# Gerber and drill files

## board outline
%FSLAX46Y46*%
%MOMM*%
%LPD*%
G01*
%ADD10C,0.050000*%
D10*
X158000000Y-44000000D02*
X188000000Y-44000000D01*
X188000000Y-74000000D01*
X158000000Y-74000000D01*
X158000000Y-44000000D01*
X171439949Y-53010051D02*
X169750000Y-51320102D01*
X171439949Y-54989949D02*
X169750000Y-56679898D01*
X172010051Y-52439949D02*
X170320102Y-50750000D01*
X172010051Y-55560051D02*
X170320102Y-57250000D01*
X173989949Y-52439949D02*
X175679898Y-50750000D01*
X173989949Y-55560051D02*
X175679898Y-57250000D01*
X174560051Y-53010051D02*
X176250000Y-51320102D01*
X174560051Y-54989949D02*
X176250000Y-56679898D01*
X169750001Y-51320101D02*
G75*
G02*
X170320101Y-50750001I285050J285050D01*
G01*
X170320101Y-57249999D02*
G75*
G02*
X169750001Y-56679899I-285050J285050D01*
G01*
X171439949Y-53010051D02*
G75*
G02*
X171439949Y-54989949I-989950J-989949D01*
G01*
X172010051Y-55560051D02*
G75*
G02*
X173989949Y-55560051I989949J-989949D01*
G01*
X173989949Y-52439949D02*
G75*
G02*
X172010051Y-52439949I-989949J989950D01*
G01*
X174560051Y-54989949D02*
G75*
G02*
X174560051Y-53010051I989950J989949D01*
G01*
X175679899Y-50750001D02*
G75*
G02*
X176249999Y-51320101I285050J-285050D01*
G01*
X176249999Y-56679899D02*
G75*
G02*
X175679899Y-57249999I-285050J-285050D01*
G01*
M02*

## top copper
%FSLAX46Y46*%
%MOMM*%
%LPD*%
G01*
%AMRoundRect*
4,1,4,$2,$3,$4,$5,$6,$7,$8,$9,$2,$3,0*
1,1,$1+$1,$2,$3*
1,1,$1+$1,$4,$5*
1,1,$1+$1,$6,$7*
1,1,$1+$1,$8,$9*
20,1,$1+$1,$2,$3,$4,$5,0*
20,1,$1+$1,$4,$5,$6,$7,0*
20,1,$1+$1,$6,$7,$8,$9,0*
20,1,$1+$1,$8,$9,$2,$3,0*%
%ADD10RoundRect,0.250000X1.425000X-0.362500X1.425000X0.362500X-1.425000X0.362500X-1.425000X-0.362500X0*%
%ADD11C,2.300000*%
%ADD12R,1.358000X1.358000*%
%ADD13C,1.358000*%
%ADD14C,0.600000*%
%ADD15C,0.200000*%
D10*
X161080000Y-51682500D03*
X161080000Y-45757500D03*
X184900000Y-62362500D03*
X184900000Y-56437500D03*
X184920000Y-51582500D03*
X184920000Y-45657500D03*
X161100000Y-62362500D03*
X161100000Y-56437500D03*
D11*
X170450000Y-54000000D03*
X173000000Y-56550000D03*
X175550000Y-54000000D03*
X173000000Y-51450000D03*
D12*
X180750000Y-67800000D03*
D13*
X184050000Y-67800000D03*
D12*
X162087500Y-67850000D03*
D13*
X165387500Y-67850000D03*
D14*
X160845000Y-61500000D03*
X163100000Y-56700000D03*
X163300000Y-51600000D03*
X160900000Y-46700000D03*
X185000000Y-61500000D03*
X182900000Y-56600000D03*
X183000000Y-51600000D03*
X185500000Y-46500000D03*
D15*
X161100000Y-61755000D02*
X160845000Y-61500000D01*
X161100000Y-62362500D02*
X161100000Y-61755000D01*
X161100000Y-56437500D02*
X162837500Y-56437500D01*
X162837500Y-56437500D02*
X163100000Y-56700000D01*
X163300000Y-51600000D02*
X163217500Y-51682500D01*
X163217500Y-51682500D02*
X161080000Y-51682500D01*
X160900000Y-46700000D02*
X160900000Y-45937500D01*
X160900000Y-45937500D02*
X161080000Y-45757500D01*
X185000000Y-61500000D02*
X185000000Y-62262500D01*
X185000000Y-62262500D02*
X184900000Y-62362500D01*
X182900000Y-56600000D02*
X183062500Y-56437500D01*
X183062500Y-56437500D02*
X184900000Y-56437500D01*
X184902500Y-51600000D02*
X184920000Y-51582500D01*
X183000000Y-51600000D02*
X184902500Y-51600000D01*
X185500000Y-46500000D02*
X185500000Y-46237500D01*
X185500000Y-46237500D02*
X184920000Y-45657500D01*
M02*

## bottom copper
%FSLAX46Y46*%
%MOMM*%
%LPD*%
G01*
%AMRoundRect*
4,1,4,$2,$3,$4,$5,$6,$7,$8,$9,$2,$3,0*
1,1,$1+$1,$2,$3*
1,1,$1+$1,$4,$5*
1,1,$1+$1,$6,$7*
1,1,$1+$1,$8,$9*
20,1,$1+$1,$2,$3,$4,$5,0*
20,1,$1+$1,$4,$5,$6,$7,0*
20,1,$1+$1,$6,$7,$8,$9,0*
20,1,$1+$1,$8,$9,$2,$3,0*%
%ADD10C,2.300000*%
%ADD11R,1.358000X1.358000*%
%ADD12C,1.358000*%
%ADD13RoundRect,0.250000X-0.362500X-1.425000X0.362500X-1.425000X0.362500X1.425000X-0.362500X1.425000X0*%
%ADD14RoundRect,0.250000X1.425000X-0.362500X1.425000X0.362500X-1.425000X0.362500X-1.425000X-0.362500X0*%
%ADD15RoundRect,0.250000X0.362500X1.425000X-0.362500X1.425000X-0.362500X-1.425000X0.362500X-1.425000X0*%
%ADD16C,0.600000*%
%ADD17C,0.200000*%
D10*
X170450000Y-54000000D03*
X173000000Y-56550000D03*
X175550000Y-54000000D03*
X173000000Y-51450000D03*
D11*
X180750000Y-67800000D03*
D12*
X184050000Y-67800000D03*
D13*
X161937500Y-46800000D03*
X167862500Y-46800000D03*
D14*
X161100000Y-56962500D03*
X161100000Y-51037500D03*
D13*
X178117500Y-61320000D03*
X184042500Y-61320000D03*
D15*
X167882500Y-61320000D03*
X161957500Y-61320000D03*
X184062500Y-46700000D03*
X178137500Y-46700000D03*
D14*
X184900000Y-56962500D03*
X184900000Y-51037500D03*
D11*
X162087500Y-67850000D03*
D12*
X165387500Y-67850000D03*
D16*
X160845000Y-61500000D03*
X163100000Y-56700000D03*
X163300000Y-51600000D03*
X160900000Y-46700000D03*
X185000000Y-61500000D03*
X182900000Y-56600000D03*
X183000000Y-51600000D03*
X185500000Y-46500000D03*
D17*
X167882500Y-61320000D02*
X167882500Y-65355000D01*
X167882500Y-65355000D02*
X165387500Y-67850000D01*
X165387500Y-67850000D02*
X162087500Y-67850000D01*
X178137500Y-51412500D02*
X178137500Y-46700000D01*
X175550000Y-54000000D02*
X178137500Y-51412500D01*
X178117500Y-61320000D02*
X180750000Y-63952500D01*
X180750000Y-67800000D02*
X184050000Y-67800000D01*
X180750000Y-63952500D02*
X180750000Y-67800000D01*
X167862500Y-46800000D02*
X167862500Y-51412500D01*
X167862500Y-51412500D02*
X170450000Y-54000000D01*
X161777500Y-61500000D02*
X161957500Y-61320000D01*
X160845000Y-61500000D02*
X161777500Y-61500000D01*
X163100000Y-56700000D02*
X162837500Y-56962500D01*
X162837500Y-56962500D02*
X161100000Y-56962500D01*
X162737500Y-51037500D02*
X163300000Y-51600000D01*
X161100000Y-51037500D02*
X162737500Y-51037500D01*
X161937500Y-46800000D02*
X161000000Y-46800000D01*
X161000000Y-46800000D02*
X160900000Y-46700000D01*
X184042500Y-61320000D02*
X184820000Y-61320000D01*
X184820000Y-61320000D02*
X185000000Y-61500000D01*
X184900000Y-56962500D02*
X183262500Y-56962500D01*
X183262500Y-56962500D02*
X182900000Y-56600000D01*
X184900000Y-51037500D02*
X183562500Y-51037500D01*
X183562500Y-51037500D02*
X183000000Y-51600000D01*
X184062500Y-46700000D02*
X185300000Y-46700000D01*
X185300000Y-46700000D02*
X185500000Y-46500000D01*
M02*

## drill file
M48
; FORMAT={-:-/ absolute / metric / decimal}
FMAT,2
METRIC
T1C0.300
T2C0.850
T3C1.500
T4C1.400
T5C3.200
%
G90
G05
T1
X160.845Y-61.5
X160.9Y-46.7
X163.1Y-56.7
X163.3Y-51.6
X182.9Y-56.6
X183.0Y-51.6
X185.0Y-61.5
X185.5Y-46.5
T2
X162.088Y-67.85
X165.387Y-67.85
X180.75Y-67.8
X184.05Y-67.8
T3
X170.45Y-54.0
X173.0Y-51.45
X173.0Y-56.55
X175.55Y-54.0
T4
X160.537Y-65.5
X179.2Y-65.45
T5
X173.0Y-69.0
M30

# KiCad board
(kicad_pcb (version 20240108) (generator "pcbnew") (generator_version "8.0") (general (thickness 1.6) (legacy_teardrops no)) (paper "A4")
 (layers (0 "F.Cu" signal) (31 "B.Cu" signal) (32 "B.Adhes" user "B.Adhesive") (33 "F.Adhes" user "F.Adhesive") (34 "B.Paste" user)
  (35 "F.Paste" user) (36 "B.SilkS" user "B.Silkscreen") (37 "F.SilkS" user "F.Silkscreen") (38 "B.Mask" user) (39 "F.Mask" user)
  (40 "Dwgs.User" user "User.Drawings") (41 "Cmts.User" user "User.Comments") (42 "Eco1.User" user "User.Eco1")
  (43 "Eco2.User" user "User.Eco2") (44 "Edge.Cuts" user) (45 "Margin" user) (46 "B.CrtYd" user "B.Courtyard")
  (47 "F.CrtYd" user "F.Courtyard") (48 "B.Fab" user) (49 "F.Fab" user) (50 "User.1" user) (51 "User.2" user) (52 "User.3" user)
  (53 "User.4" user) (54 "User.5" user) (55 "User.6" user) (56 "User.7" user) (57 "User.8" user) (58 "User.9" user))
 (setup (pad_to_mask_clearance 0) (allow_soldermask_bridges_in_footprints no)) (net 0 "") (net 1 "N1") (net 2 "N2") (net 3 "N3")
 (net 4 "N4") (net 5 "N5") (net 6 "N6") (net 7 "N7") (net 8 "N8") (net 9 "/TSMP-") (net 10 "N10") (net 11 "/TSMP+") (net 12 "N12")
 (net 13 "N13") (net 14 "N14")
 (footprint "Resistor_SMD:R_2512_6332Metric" (layer "F.Cu") (at 161.08 48.72 90)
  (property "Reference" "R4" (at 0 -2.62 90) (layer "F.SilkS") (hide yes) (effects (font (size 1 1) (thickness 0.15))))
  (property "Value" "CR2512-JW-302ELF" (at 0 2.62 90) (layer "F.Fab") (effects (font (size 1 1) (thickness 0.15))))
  (pad "1" smd roundrect (at -2.9625 0 90) (size 1.225 3.35) (layers "F.Cu" "F.Paste" "F.Mask") (roundrect_rratio 0.204082) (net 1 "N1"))
  (pad "2" smd roundrect (at 2.9625 0 90) (size 1.225 3.35) (layers "F.Cu" "F.Paste" "F.Mask") (roundrect_rratio 0.204082) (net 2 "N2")))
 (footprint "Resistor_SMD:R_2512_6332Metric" (layer "F.Cu") (at 184.9 59.4 90)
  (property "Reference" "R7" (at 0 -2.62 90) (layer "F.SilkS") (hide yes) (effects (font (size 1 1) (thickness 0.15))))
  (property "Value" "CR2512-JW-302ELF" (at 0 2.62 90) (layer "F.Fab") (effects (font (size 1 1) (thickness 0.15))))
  (pad "1" smd roundrect (at -2.9625 0 90) (size 1.225 3.35) (layers "F.Cu" "F.Paste" "F.Mask") (roundrect_rratio 0.204082) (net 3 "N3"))
  (pad "2" smd roundrect (at 2.9625 0 90) (size 1.225 3.35) (layers "F.Cu" "F.Paste" "F.Mask") (roundrect_rratio 0.204082) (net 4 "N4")))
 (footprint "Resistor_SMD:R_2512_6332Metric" (layer "F.Cu") (at 184.92 48.62 90)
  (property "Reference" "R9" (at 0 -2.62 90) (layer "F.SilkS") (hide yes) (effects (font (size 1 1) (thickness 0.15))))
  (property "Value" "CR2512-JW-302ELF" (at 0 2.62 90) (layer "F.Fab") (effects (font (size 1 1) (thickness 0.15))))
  (pad "1" smd roundrect (at -2.9625 0 90) (size 1.225 3.35) (layers "F.Cu" "F.Paste" "F.Mask") (roundrect_rratio 0.204082) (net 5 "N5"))
  (pad "2" smd roundrect (at 2.9625 0 90) (size 1.225 3.35) (layers "F.Cu" "F.Paste" "F.Mask") (roundrect_rratio 0.204082) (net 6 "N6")))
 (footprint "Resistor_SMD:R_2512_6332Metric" (layer "F.Cu") (at 161.1 59.4 90)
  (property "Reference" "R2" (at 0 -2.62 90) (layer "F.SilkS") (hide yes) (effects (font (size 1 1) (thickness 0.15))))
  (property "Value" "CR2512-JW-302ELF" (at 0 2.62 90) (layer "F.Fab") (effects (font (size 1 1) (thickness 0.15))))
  (pad "1" smd roundrect (at -2.9625 0 90) (size 1.225 3.35) (layers "F.Cu" "F.Paste" "F.Mask") (roundrect_rratio 0.204082) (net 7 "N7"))
  (pad "2" smd roundrect (at 2.9625 0 90) (size 1.225 3.35) (layers "F.Cu" "F.Paste" "F.Mask") (roundrect_rratio 0.204082) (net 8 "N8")))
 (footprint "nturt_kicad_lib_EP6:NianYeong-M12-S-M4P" (layer "F.Cu") (at 173 54 -90)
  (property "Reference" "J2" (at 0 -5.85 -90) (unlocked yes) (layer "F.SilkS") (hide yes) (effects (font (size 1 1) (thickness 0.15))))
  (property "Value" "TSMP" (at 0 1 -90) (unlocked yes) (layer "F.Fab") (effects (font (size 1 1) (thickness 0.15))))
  (fp_line (start -0.989949 1.560051) (end -2.679898 3.25) (stroke (width 0.05) (type default)) (layer "Edge.Cuts"))
  (fp_line (start 0.989949 1.560051) (end 2.679898 3.25) (stroke (width 0.05) (type default)) (layer "Edge.Cuts"))
  (fp_line (start -1.560051 0.989949) (end -3.25 2.679898) (stroke (width 0.05) (type default)) (layer "Edge.Cuts"))
  (fp_line (start 1.560051 0.989949) (end 3.25 2.679898) (stroke (width 0.05) (type default)) (layer "Edge.Cuts"))
  (fp_line (start -1.560051 -0.989949) (end -3.25 -2.679898) (stroke (width 0.05) (type default)) (layer "Edge.Cuts"))
  (fp_line (start 1.560051 -0.989949) (end 3.25 -2.679898) (stroke (width 0.05) (type default)) (layer "Edge.Cuts"))
  (fp_line (start -0.989949 -1.560051) (end -2.679898 -3.25) (stroke (width 0.05) (type default)) (layer "Edge.Cuts"))
  (fp_line (start 0.989949 -1.560051) (end 2.679898 -3.25) (stroke (width 0.05) (type default)) (layer "Edge.Cuts"))
  (fp_arc (start -2.679899 3.249999) (mid -3.249999 3.249999) (end -3.249999 2.679899) (stroke (width 0.05) (type default))
   (layer "Edge.Cuts"))
  (fp_arc (start 3.249999 2.679899) (mid 3.249999 3.249999) (end 2.679899 3.249999) (stroke (width 0.05) (type default)) (layer "Edge.Cuts"))
  (fp_arc (start -0.989949 1.560051) (mid 0 1.150001) (end 0.989949 1.560051) (stroke (width 0.05) (type default)) (layer "Edge.Cuts"))
  (fp_arc (start 1.560051 0.989949) (mid 1.150001 0) (end 1.560051 -0.989949) (stroke (width 0.05) (type default)) (layer "Edge.Cuts"))
  (fp_arc (start -1.560051 -0.989949) (mid -1.150001 0) (end -1.560051 0.989949) (stroke (width 0.05) (type default)) (layer "Edge.Cuts"))
  (fp_arc (start 0.989949 -1.560051) (mid 0 -1.150001) (end -0.989949 -1.560051) (stroke (width 0.05) (type default)) (layer "Edge.Cuts"))
  (fp_arc (start -3.249999 -2.679899) (mid -3.249999 -3.249999) (end -2.679899 -3.249999) (stroke (width 0.05) (type default))
   (layer "Edge.Cuts"))
  (fp_arc (start 2.679899 -3.249999) (mid 3.249999 -3.249999) (end 3.249999 -2.679899) (stroke (width 0.05) (type default))
   (layer "Edge.Cuts"))
  (pad "1" thru_hole circle (at 0 2.55 270) (size 2.3 2.3) (drill 1.5) (layers "*.Cu" "*.Mask") (remove_unused_layers no) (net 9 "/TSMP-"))
  (pad "2" thru_hole circle (at 2.55 0 270) (size 2.3 2.3) (drill 1.5) (layers "*.Cu" "*.Mask") (remove_unused_layers no) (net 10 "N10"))
  (pad "3" thru_hole circle (at 0 -2.55 270) (size 2.3 2.3) (drill 1.5) (layers "*.Cu" "*.Mask") (remove_unused_layers no) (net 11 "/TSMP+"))
  (pad "4" thru_hole circle (at -2.55 0 270) (size 2.3 2.3) (drill 1.5) (layers "*.Cu" "*.Mask") (remove_unused_layers no) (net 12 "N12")))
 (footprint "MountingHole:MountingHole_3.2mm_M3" (layer "F.Cu") (at 173 69)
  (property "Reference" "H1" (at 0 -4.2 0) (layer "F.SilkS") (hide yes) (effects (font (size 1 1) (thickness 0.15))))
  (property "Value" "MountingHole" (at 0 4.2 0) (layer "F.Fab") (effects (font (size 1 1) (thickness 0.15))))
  (pad "" np_thru_hole circle (at 0 0) (size 3.2 3.2) (drill 3.2) (layers "*.Cu" "*.Mask")))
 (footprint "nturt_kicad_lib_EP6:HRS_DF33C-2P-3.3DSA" (layer "B.Cu") (at 182.4 67.8 180)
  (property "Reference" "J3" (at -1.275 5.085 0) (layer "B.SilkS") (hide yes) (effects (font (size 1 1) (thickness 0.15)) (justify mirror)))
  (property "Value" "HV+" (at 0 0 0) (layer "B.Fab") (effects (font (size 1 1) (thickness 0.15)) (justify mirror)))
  (pad "" np_thru_hole circle (at 3.2 2.35 180) (size 1.4 1.4) (drill 1.4) (layers "*.Cu" "*.Mask"))
  (pad "1" thru_hole rect (at 1.65 0 180) (size 1.358 1.358) (drill 0.85) (layers "*.Cu" "*.Mask") (remove_unused_layers no) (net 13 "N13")
   (solder_mask_margin 0.102))
  (pad "2" thru_hole circle (at -1.65 0 180) (size 1.358 1.358) (drill 0.85) (layers "*.Cu" "*.Mask") (remove_unused_layers no)
   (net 13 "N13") (solder_mask_margin 0.102)))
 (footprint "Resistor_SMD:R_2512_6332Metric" (layer "B.Cu") (at 164.9 46.8)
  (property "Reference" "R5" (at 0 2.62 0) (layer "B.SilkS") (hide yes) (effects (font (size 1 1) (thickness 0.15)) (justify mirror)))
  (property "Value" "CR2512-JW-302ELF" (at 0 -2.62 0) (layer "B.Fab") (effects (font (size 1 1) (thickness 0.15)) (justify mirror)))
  (pad "1" smd roundrect (at -2.9625 0) (size 1.225 3.35) (layers "B.Cu" "B.Paste" "B.Mask") (roundrect_rratio 0.204082) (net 2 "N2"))
  (pad "2" smd roundrect (at 2.9625 0) (size 1.225 3.35) (layers "B.Cu" "B.Paste" "B.Mask") (roundrect_rratio 0.204082) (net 9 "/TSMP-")))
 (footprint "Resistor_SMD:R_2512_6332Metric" (layer "B.Cu") (at 161.1 54 90)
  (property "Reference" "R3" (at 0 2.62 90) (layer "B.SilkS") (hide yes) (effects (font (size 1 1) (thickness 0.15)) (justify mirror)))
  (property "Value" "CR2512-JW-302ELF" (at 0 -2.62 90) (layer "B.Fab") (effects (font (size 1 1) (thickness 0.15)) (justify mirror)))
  (pad "1" smd roundrect (at -2.9625 0 90) (size 1.225 3.35) (layers "B.Cu" "B.Paste" "B.Mask") (roundrect_rratio 0.204082) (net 8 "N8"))
  (pad "2" smd roundrect (at 2.9625 0 90) (size 1.225 3.35) (layers "B.Cu" "B.Paste" "B.Mask") (roundrect_rratio 0.204082) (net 1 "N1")))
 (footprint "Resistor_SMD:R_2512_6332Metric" (layer "B.Cu") (at 181.08 61.32)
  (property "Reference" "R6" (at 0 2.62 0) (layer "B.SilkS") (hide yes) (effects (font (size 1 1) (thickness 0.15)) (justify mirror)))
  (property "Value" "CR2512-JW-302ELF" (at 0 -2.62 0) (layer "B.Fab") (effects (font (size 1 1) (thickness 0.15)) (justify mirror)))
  (pad "1" smd roundrect (at -2.9625 0) (size 1.225 3.35) (layers "B.Cu" "B.Paste" "B.Mask") (roundrect_rratio 0.204082) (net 13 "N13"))
  (pad "2" smd roundrect (at 2.9625 0) (size 1.225 3.35) (layers "B.Cu" "B.Paste" "B.Mask") (roundrect_rratio 0.204082) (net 3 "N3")))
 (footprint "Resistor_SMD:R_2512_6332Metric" (layer "B.Cu") (at 164.92 61.32 180)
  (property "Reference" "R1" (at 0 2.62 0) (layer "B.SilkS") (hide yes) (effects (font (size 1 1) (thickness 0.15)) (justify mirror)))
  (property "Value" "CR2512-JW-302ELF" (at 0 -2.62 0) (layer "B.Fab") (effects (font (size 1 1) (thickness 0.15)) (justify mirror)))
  (pad "1" smd roundrect (at -2.9625 0 180) (size 1.225 3.35) (layers "B.Cu" "B.Paste" "B.Mask") (roundrect_rratio 0.204082) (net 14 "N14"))
  (pad "2" smd roundrect (at 2.9625 0 180) (size 1.225 3.35) (layers "B.Cu" "B.Paste" "B.Mask") (roundrect_rratio 0.204082) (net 7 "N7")))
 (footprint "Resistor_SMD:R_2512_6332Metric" (layer "B.Cu") (at 181.1 46.7 180)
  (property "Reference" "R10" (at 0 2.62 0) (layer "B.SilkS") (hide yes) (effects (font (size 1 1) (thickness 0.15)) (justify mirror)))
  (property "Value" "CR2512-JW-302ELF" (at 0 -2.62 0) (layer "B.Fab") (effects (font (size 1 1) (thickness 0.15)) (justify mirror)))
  (pad "1" smd roundrect (at -2.9625 0 180) (size 1.225 3.35) (layers "B.Cu" "B.Paste" "B.Mask") (roundrect_rratio 0.204082) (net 6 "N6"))
  (pad "2" smd roundrect (at 2.9625 0 180) (size 1.225 3.35) (layers "B.Cu" "B.Paste" "B.Mask") (roundrect_rratio 0.204082)
   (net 11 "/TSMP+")))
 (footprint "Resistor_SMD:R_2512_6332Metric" (layer "B.Cu") (at 184.9 54 90)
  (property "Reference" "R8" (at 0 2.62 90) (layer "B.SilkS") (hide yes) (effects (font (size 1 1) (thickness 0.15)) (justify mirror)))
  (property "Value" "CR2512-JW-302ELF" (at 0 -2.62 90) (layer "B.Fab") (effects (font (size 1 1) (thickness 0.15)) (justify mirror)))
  (pad "1" smd roundrect (at -2.9625 0 90) (size 1.225 3.35) (layers "B.Cu" "B.Paste" "B.Mask") (roundrect_rratio 0.204082) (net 4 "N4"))
  (pad "2" smd roundrect (at 2.9625 0 90) (size 1.225 3.35) (layers "B.Cu" "B.Paste" "B.Mask") (roundrect_rratio 0.204082) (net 5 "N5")))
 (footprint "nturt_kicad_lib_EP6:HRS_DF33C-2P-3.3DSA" (layer "B.Cu") (at 163.7375 67.85 180)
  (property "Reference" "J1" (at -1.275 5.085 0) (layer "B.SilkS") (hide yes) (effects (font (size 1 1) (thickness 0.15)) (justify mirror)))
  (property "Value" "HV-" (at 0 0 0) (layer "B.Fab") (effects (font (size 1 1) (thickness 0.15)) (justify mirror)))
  (pad "" np_thru_hole circle (at 3.2 2.35 180) (size 1.4 1.4) (drill 1.4) (layers "*.Cu" "*.Mask"))
  (pad "1" thru_hole rect (at 1.65 0 180) (size 1.358 1.358) (drill 0.85) (layers "*.Cu" "*.Mask") (remove_unused_layers no) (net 14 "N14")
   (solder_mask_margin 0.102))
  (pad "2" thru_hole circle (at -1.65 0 180) (size 1.358 1.358) (drill 0.85) (layers "*.Cu" "*.Mask") (remove_unused_layers no)
   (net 14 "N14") (solder_mask_margin 0.102)))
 (gr_rect (start 158 44) (end 188 74) (stroke (width 0.05) (type default)) (fill none) (layer "Edge.Cuts"))
 (segment (start 167.8825 61.32) (end 167.8825 65.355) (width 0.2) (layer "B.Cu") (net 14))
 (segment (start 167.8825 65.355) (end 165.3875 67.85) (width 0.2) (layer "B.Cu") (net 14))
 (segment (start 165.3875 67.85) (end 162.0875 67.85) (width 0.2) (layer "B.Cu") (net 14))
 (segment (start 178.1375 51.4125) (end 178.1375 46.7) (width 0.2) (layer "B.Cu") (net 11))
 (segment (start 175.55 54) (end 178.1375 51.4125) (width 0.2) (layer "B.Cu") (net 11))
 (segment (start 178.1175 61.32) (end 180.75 63.9525) (width 0.2) (layer "B.Cu") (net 13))
 (segment (start 180.75 67.8) (end 184.05 67.8) (width 0.2) (layer "B.Cu") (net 13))
 (segment (start 180.75 63.9525) (end 180.75 67.8) (width 0.2) (layer "B.Cu") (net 13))
 (segment (start 167.8625 46.8) (end 167.8625 51.4125) (width 0.2) (layer "B.Cu") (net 9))
 (segment (start 167.8625 51.4125) (end 170.45 54) (width 0.2) (layer "B.Cu") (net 9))
 (segment (start 161.1 61.755) (end 160.845 61.5) (width 0.2) (layer "F.Cu") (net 7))
 (segment (start 161.1 62.3625) (end 161.1 61.755) (width 0.2) (layer "F.Cu") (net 7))
 (via (at 160.845 61.5) (size 0.6) (drill 0.3) (layers "F.Cu" "B.Cu") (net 7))
 (segment (start 161.7775 61.5) (end 161.9575 61.32) (width 0.2) (layer "B.Cu") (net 7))
 (segment (start 160.845 61.5) (end 161.7775 61.5) (width 0.2) (layer "B.Cu") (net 7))
 (segment (start 161.1 56.4375) (end 162.8375 56.4375) (width 0.2) (layer "F.Cu") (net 8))
 (segment (start 162.8375 56.4375) (end 163.1 56.7) (width 0.2) (layer "F.Cu") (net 8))
 (via (at 163.1 56.7) (size 0.6) (drill 0.3) (layers "F.Cu" "B.Cu") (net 8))
 (segment (start 163.1 56.7) (end 162.8375 56.9625) (width 0.2) (layer "B.Cu") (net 8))
 (segment (start 162.8375 56.9625) (end 161.1 56.9625) (width 0.2) (layer "B.Cu") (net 8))
 (segment (start 163.3 51.6) (end 163.2175 51.6825) (width 0.2) (layer "F.Cu") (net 1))
 (segment (start 163.2175 51.6825) (end 161.08 51.6825) (width 0.2) (layer "F.Cu") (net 1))
 (via (at 163.3 51.6) (size 0.6) (drill 0.3) (layers "F.Cu" "B.Cu") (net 1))
 (segment (start 162.7375 51.0375) (end 163.3 51.6) (width 0.2) (layer "B.Cu") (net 1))
 (segment (start 161.1 51.0375) (end 162.7375 51.0375) (width 0.2) (layer "B.Cu") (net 1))
 (segment (start 160.9 46.7) (end 160.9 45.9375) (width 0.2) (layer "F.Cu") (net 2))
 (segment (start 160.9 45.9375) (end 161.08 45.7575) (width 0.2) (layer "F.Cu") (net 2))
 (via (at 160.9 46.7) (size 0.6) (drill 0.3) (layers "F.Cu" "B.Cu") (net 2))
 (segment (start 161.9375 46.8) (end 161 46.8) (width 0.2) (layer "B.Cu") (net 2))
 (segment (start 161 46.8) (end 160.9 46.7) (width 0.2) (layer "B.Cu") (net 2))
 (segment (start 185 61.5) (end 185 62.2625) (width 0.2) (layer "F.Cu") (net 3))
 (segment (start 185 62.2625) (end 184.9 62.3625) (width 0.2) (layer "F.Cu") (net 3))
 (via (at 185 61.5) (size 0.6) (drill 0.3) (layers "F.Cu" "B.Cu") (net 3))
 (segment (start 184.0425 61.32) (end 184.82 61.32) (width 0.2) (layer "B.Cu") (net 3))
 (segment (start 184.82 61.32) (end 185 61.5) (width 0.2) (layer "B.Cu") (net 3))
 (segment (start 182.9 56.6) (end 183.0625 56.4375) (width 0.2) (layer "F.Cu") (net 4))
 (segment (start 183.0625 56.4375) (end 184.9 56.4375) (width 0.2) (layer "F.Cu") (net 4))
 (via (at 182.9 56.6) (size 0.6) (drill 0.3) (layers "F.Cu" "B.Cu") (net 4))
 (segment (start 184.9 56.9625) (end 183.2625 56.9625) (width 0.2) (layer "B.Cu") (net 4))
 (segment (start 183.2625 56.9625) (end 182.9 56.6) (width 0.2) (layer "B.Cu") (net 4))
 (segment (start 184.9025 51.6) (end 184.92 51.5825) (width 0.2) (layer "F.Cu") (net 5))
 (segment (start 183 51.6) (end 184.9025 51.6) (width 0.2) (layer "F.Cu") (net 5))
 (via (at 183 51.6) (size 0.6) (drill 0.3) (layers "F.Cu" "B.Cu") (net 5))
 (segment (start 184.9 51.0375) (end 183.5625 51.0375) (width 0.2) (layer "B.Cu") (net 5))
 (segment (start 183.5625 51.0375) (end 183 51.6) (width 0.2) (layer "B.Cu") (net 5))
 (segment (start 185.5 46.5) (end 185.5 46.2375) (width 0.2) (layer "F.Cu") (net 6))
 (segment (start 185.5 46.2375) (end 184.92 45.6575) (width 0.2) (layer "F.Cu") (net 6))
 (via (at 185.5 46.5) (size 0.6) (drill 0.3) (layers "F.Cu" "B.Cu") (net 6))
 (segment (start 184.0625 46.7) (end 185.3 46.7) (width 0.2) (layer "B.Cu") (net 6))
 (segment (start 185.3 46.7) (end 185.5 46.5) (width 0.2) (layer "B.Cu") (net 6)))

